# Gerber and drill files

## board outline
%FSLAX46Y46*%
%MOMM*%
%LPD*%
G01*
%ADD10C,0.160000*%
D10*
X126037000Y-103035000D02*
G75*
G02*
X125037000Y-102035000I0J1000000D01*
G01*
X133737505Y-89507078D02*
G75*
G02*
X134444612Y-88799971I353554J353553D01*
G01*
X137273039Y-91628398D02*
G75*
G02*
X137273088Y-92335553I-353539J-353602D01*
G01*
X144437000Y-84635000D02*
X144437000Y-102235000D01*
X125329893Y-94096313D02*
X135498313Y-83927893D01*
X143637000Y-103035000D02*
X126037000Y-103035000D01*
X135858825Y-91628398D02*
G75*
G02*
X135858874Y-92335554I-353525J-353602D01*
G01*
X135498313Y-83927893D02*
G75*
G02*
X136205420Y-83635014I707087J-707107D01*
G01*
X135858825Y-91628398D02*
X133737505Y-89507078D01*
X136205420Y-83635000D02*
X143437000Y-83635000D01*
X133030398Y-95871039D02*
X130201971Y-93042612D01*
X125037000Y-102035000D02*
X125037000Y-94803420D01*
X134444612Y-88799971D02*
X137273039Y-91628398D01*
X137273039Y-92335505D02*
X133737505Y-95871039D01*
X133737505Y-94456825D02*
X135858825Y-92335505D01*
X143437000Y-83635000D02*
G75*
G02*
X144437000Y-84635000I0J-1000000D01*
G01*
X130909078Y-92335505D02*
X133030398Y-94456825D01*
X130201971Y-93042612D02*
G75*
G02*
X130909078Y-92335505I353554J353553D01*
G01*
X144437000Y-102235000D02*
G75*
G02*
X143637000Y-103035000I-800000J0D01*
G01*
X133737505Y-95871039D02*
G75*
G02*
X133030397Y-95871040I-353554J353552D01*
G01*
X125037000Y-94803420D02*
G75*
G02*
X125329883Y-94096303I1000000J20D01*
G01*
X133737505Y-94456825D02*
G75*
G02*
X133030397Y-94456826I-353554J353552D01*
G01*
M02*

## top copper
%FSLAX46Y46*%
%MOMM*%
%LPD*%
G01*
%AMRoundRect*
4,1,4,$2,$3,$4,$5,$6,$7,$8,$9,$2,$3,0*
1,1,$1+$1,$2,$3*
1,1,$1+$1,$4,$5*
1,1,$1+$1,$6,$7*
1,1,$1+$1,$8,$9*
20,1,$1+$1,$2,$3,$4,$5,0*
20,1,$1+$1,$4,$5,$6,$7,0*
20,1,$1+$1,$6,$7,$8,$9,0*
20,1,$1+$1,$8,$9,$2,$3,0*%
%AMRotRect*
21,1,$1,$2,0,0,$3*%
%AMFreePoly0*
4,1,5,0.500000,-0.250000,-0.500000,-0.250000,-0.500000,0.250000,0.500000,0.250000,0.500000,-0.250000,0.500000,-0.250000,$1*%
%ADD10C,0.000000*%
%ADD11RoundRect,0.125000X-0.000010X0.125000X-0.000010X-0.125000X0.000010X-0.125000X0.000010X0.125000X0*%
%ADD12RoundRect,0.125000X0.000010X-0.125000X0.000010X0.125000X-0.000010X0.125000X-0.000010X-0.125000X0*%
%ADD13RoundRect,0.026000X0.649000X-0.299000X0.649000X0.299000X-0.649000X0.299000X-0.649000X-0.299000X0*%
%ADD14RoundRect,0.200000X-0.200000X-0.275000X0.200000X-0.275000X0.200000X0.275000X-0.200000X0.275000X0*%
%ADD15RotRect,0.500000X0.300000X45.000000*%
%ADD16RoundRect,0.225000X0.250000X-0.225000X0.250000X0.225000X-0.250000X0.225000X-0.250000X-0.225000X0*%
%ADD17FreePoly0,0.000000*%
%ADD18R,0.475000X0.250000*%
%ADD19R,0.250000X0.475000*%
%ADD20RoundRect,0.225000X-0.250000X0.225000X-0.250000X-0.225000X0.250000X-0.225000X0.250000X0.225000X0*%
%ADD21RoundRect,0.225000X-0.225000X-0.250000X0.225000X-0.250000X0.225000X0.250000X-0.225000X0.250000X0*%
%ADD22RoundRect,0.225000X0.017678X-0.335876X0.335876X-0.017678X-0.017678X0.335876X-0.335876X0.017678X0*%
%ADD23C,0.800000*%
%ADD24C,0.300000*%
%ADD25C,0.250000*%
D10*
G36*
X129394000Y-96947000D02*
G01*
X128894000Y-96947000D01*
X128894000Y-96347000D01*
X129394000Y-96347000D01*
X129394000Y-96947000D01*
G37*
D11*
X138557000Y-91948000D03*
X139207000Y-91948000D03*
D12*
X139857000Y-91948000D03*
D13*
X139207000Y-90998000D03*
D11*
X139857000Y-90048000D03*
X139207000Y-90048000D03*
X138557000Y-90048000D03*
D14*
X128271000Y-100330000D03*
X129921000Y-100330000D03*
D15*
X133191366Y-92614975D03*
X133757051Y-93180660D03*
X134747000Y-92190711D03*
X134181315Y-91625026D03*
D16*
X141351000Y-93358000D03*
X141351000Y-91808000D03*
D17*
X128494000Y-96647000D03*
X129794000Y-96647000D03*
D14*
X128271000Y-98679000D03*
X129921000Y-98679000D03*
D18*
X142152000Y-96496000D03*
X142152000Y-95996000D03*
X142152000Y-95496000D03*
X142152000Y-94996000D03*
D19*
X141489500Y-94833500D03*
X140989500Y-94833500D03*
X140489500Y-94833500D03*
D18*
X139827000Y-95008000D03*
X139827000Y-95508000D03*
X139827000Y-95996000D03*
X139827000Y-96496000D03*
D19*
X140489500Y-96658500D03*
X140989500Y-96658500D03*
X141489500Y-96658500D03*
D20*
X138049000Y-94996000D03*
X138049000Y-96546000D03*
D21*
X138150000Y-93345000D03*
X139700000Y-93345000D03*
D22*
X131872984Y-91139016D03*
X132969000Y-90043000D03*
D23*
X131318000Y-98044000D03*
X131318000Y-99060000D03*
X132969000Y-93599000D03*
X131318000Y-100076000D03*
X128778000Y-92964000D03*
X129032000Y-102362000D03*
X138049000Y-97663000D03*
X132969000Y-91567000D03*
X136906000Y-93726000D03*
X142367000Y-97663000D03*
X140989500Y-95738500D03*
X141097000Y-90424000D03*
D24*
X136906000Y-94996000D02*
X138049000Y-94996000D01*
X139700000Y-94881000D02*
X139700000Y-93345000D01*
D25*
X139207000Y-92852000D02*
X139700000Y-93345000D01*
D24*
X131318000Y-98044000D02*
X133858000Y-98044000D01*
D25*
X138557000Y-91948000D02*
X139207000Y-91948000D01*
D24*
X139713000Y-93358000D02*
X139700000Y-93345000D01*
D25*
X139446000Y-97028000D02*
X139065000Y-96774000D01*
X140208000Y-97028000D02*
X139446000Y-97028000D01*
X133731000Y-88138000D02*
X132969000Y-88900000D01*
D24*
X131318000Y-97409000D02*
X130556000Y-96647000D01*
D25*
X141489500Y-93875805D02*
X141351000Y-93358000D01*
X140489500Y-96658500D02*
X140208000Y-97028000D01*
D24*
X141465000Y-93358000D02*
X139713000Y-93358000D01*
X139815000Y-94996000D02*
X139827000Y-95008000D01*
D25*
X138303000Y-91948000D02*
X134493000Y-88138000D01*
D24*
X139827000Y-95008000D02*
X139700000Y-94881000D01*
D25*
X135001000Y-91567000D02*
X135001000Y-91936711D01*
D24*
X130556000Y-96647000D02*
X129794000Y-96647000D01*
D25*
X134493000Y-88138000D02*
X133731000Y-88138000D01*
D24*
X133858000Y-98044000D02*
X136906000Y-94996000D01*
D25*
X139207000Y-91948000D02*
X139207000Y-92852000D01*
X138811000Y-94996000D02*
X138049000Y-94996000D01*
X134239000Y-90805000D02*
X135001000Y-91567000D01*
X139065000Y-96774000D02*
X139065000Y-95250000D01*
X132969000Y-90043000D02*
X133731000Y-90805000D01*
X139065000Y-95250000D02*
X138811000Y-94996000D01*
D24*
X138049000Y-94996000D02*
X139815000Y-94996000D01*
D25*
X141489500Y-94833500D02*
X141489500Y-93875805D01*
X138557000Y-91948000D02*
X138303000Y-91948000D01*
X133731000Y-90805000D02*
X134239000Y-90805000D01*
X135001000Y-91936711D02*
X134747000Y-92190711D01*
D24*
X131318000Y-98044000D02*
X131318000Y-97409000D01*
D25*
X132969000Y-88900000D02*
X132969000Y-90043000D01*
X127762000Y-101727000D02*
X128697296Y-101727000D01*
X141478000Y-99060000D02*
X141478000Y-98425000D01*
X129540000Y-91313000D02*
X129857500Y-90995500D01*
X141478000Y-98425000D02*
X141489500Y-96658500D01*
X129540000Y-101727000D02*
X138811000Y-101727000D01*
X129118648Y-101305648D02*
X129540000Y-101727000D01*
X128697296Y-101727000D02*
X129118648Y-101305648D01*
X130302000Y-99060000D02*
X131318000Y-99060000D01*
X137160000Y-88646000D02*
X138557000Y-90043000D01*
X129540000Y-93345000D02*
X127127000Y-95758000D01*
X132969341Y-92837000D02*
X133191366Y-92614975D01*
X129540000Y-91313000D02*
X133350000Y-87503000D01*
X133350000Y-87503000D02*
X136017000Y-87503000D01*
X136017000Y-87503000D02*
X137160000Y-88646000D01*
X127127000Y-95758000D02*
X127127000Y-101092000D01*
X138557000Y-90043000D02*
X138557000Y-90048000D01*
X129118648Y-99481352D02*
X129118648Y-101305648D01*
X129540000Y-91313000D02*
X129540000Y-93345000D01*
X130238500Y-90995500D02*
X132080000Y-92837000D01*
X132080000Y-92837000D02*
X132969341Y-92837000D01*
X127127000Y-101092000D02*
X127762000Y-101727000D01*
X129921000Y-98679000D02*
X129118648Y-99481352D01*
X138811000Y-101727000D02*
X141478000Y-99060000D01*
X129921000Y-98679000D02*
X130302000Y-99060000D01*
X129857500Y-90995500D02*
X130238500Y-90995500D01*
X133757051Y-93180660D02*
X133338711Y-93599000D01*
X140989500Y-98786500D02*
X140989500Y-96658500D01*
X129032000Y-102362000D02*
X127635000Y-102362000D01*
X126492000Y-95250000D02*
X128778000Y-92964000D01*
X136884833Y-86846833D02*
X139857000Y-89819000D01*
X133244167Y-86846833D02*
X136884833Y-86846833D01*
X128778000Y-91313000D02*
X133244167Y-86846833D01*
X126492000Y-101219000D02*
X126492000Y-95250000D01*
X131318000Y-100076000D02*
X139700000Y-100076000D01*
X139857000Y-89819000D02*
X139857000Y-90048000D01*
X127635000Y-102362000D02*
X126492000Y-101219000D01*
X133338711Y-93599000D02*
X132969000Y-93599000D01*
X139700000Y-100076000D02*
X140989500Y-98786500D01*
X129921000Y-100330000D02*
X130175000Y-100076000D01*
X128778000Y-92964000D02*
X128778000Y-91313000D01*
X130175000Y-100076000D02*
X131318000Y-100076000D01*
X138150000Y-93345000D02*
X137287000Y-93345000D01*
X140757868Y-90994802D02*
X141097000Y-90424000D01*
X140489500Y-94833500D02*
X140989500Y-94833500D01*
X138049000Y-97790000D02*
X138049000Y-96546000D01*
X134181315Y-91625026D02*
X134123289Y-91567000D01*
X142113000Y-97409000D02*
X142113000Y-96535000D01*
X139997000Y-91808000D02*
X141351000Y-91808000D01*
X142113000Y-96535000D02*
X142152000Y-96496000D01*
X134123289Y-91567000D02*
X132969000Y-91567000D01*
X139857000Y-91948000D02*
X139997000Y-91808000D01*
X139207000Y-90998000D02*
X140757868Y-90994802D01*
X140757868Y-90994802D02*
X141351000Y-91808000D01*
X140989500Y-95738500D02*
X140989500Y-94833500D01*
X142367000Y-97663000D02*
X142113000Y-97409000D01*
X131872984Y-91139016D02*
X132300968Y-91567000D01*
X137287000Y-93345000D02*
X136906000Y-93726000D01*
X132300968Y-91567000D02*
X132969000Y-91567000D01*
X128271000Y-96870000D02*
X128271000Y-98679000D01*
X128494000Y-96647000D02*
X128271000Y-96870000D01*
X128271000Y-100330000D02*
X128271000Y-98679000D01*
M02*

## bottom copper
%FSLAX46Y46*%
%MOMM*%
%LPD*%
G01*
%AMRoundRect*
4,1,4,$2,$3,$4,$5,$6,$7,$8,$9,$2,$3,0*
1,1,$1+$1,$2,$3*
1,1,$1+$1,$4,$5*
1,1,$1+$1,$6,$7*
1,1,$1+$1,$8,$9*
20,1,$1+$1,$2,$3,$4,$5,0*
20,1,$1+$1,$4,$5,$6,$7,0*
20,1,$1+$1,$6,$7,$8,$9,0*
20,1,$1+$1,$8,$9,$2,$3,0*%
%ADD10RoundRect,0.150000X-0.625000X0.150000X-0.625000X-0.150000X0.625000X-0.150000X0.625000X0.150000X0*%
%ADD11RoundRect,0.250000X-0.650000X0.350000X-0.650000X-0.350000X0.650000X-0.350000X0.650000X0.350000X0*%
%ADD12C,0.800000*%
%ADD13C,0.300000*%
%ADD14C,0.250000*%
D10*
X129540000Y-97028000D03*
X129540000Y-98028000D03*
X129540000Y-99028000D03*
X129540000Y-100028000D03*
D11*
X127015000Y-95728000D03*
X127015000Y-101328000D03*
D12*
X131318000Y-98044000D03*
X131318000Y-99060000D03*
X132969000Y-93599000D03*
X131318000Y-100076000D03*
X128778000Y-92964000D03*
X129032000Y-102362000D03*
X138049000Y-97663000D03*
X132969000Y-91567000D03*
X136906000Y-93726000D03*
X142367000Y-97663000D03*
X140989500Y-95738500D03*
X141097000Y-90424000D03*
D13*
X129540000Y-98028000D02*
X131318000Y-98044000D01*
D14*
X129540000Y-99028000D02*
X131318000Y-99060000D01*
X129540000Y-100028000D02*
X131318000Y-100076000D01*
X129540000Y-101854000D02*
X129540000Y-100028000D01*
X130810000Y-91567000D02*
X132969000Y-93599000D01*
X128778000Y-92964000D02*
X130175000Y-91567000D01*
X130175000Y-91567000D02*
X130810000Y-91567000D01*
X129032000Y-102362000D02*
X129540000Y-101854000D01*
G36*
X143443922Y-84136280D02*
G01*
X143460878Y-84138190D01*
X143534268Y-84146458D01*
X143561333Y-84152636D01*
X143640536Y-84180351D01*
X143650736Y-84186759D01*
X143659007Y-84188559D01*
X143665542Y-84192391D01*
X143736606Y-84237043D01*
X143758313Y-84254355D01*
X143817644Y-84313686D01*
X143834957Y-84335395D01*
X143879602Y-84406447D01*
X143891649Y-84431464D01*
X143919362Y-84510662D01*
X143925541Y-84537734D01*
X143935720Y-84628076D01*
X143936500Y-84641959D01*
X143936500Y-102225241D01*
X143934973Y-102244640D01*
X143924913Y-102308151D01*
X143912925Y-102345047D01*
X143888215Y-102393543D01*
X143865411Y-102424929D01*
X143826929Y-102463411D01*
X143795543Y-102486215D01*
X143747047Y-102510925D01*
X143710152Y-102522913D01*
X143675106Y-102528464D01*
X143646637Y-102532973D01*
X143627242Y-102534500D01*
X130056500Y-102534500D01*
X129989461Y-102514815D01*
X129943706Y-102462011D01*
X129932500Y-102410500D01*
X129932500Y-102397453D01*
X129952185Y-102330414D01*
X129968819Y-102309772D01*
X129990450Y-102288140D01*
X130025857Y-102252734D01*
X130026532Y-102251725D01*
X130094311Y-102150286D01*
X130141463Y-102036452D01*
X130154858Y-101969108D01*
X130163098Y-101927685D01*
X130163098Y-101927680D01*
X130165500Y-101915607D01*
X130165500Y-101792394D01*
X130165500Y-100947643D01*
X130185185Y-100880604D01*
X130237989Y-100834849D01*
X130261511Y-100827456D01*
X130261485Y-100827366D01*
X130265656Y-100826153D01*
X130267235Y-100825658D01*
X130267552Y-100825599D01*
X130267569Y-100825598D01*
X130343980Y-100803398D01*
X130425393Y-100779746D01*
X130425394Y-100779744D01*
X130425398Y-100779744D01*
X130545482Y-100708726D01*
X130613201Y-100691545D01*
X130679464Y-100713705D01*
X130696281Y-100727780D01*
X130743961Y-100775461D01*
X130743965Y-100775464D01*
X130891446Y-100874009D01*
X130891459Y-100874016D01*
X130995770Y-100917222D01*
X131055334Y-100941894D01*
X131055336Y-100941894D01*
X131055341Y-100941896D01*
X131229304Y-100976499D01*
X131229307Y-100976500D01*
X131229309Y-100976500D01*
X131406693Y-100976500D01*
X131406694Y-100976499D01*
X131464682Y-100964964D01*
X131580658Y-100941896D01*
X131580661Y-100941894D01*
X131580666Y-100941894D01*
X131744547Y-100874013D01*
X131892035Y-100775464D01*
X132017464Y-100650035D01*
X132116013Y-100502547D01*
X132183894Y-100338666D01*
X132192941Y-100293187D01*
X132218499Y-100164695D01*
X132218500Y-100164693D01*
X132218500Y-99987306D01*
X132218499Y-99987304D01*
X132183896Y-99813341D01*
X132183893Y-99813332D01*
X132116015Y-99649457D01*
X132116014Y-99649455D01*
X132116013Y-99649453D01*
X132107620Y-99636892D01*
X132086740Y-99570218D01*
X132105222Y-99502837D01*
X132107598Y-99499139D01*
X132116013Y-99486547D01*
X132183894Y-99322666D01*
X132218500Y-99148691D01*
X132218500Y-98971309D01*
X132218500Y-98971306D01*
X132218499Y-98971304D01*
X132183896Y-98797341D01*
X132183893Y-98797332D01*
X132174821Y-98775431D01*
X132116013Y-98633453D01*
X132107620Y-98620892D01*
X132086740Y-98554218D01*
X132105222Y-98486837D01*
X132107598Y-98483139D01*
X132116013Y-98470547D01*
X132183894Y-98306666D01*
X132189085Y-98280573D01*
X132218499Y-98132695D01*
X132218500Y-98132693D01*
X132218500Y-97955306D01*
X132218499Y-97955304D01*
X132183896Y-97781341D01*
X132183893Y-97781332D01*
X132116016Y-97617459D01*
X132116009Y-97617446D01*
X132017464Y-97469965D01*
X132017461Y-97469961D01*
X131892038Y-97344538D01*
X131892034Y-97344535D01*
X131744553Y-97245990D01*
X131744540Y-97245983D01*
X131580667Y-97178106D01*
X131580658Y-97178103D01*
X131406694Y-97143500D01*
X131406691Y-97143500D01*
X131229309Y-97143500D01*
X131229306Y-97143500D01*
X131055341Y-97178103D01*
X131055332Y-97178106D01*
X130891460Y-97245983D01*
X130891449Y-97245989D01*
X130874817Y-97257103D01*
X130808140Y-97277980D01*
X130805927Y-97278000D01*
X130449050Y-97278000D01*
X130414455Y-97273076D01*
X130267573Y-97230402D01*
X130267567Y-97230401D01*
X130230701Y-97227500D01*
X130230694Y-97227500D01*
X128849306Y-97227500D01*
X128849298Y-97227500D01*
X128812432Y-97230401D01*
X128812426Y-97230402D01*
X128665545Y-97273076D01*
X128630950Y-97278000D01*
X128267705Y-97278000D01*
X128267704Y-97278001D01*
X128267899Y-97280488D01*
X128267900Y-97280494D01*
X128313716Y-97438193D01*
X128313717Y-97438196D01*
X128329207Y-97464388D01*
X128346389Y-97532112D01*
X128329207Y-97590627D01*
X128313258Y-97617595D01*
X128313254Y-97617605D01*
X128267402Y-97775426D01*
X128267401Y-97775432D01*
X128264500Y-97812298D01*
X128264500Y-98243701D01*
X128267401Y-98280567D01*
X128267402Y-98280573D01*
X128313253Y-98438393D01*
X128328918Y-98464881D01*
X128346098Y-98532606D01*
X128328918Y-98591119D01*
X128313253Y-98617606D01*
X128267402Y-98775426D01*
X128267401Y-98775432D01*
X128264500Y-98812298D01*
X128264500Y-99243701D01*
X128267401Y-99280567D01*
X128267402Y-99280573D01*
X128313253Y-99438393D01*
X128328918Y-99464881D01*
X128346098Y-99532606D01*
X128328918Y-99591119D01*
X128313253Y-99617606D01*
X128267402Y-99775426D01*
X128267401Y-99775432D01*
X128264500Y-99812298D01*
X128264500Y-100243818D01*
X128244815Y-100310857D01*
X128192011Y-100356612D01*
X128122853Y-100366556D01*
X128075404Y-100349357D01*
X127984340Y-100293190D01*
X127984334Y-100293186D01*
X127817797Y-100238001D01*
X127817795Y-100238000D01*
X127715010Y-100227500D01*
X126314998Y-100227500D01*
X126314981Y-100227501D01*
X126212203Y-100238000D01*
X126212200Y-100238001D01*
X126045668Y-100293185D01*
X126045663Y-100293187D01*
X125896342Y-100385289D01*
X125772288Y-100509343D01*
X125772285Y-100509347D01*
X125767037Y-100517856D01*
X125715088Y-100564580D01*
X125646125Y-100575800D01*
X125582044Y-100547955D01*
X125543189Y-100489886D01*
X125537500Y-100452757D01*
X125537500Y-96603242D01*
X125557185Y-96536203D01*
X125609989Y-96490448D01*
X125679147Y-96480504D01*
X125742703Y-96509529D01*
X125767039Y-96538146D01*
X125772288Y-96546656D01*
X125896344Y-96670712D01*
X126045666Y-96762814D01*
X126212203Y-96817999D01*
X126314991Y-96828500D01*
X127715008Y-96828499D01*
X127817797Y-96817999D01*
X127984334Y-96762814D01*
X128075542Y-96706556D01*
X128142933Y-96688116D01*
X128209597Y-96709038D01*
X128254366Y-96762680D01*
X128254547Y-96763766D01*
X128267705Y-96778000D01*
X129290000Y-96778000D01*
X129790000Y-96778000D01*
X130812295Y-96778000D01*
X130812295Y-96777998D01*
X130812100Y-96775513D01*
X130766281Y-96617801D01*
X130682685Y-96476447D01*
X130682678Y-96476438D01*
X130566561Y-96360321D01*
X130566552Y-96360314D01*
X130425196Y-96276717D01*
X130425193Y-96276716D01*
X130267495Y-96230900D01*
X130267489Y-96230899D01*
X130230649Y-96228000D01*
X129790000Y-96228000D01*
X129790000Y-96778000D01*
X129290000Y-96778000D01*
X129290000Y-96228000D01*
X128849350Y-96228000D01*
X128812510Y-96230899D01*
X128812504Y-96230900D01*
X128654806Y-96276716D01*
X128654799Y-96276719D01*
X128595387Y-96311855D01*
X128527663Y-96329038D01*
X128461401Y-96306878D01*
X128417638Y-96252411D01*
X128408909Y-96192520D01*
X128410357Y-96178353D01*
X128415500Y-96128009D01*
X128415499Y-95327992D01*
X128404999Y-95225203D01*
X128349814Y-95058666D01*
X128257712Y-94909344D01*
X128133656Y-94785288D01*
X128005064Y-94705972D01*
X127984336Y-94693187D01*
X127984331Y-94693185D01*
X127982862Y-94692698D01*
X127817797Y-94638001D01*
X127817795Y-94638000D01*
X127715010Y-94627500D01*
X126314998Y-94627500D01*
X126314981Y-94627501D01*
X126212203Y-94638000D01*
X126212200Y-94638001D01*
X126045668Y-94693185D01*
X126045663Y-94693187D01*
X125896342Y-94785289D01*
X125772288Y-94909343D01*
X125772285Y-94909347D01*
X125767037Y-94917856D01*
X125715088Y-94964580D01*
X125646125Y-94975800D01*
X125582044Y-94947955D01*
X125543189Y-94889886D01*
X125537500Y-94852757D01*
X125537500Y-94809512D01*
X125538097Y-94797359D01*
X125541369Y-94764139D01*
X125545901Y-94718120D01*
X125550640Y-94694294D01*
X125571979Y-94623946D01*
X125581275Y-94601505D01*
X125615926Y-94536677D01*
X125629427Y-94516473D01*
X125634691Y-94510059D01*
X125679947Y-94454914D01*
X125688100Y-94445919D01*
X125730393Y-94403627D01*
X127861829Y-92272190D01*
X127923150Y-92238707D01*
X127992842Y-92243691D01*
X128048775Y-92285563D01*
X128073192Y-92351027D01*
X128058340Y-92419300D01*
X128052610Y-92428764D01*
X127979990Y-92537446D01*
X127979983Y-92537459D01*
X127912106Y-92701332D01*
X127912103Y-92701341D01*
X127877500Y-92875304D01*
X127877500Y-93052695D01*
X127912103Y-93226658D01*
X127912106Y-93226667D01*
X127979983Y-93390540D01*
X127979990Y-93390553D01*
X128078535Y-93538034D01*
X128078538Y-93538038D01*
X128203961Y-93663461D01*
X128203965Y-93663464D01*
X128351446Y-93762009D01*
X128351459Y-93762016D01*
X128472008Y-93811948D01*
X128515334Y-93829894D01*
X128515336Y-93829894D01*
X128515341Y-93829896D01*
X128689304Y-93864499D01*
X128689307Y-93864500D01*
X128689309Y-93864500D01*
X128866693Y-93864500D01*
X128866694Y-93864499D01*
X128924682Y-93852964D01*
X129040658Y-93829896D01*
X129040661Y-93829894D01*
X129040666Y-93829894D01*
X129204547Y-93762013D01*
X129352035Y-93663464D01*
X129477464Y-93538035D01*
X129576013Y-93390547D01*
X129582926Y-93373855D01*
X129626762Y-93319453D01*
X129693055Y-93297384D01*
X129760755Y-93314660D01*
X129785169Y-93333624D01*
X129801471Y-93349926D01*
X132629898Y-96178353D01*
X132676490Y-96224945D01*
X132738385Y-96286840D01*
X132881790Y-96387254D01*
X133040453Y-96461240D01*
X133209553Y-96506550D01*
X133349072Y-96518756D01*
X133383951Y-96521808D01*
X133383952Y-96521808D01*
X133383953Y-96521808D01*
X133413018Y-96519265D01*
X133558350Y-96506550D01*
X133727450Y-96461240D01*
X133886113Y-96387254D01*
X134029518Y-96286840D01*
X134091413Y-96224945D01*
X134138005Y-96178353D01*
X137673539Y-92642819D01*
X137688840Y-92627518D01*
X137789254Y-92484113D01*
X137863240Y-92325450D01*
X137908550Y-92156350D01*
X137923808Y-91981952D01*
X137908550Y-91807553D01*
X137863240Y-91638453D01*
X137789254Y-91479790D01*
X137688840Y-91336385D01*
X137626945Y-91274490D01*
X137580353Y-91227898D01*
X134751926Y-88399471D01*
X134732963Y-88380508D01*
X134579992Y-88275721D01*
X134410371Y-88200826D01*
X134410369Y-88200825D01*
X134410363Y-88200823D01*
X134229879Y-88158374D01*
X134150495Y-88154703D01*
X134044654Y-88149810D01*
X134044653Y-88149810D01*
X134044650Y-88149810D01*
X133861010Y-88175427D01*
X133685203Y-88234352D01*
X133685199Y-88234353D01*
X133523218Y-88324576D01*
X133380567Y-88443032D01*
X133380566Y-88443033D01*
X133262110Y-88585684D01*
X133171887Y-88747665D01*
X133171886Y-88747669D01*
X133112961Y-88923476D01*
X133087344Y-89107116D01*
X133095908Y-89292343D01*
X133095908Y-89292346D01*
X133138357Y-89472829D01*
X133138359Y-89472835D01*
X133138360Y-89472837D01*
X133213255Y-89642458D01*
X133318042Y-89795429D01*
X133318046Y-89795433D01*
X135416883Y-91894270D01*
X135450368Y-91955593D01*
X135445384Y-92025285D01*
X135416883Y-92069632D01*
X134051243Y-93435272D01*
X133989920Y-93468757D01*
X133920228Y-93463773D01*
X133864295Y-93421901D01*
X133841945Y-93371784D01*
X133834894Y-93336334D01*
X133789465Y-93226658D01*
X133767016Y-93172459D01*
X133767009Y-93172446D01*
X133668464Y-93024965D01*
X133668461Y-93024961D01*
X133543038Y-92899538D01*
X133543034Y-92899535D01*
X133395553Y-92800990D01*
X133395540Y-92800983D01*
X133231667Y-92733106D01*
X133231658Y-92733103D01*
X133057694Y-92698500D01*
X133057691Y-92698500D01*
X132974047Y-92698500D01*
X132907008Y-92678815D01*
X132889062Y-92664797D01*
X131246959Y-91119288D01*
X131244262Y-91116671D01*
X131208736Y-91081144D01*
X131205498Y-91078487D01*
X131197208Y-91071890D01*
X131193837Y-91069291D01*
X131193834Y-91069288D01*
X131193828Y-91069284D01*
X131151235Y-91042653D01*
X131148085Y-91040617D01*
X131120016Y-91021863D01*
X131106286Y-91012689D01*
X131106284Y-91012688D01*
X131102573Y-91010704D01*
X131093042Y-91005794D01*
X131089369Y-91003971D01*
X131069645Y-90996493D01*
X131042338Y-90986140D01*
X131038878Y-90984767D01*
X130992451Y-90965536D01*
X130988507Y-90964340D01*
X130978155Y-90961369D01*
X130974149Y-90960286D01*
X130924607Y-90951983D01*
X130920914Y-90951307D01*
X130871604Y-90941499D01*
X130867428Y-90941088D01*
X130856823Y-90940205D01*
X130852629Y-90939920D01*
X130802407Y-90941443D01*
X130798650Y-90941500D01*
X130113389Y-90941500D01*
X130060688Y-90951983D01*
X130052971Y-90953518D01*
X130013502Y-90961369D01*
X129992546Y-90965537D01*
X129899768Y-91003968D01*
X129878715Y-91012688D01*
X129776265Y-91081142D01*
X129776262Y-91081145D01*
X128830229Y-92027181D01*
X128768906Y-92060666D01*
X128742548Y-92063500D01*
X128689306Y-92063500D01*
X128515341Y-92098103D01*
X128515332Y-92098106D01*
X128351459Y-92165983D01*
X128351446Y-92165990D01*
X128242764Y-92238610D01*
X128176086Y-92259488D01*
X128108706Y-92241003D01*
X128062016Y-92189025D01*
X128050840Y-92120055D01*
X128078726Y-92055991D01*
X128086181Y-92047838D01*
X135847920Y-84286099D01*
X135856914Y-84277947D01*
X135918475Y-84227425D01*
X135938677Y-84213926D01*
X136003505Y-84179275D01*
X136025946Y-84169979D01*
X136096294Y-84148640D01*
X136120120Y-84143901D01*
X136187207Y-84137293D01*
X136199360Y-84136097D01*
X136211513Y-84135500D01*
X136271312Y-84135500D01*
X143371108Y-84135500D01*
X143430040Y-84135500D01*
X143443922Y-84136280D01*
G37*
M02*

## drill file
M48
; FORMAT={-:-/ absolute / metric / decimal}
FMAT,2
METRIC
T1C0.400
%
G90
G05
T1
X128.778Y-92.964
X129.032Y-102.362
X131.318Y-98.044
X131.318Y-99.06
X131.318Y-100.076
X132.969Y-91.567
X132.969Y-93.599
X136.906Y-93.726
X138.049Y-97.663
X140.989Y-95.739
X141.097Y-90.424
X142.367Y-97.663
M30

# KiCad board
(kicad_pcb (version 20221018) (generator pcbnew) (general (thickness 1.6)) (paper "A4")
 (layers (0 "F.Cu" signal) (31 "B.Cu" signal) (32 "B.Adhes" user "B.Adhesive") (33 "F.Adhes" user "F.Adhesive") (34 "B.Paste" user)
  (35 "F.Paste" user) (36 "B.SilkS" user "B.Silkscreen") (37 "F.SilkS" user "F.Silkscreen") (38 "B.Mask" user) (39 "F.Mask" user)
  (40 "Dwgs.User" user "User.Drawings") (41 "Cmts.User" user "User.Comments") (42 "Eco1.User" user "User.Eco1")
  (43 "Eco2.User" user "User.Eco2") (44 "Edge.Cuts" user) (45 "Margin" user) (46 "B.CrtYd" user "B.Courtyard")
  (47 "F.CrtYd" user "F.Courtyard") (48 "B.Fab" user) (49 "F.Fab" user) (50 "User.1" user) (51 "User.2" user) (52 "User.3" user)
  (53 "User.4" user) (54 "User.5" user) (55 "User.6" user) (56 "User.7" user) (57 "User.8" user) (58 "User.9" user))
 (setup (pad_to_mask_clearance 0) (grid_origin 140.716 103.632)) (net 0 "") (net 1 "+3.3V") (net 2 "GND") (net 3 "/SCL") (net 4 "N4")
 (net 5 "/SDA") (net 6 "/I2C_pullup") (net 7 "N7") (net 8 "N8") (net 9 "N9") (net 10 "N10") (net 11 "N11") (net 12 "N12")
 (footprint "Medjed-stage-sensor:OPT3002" (layer "F.Cu") (at 139.207 90.998 90)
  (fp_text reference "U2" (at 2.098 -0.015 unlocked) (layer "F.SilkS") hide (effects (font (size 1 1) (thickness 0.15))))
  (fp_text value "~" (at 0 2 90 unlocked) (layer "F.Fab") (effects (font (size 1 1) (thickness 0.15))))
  (pad "1" smd roundrect (at -0.95 -0.65 270) (size 0.5 0.25) (layers "F.Cu" "F.Paste" "F.Mask") (roundrect_rratio 0.5) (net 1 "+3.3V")
   (thermal_bridge_angle 45))
  (pad "2" smd roundrect (at -0.95 0 270) (size 0.5 0.25) (layers "F.Cu" "F.Paste" "F.Mask") (roundrect_rratio 0.5) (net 1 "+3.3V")
   (thermal_bridge_angle 45))
  (pad "3" smd roundrect (at -0.95 0.65 90) (size 0.5 0.25) (layers "F.Cu" "F.Paste" "F.Mask") (roundrect_rratio 0.5) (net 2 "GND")
   (thermal_bridge_angle 45))
  (pad "3" smd roundrect (at 0 0 90) (size 0.65 1.35) (layers "F.Cu" "F.Paste" "F.Mask") (roundrect_rratio 0.04) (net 2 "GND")
   (thermal_bridge_angle 45))
  (pad "4" smd roundrect (at 0.95 0.65 270) (size 0.5 0.25) (layers "F.Cu" "F.Paste" "F.Mask") (roundrect_rratio 0.5) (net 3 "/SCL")
   (thermal_bridge_angle 45))
  (pad "5" smd roundrect (at 0.95 0 270) (size 0.5 0.25) (layers "F.Cu" "F.Paste" "F.Mask") (roundrect_rratio 0.5) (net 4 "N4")
   (thermal_bridge_angle 45))
  (pad "6" smd roundrect (at 0.95 -0.65 270) (size 0.5 0.25) (layers "F.Cu" "F.Paste" "F.Mask") (roundrect_rratio 0.5) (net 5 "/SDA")
   (thermal_bridge_angle 45)))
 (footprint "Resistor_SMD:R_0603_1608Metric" (layer "F.Cu") (at 129.096 100.33)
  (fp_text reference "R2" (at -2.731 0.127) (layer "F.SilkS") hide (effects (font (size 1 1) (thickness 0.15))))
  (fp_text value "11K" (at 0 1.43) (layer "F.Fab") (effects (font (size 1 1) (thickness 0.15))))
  (pad "1" smd roundrect (at -0.825 0) (size 0.8 0.95) (layers "F.Cu" "F.Paste" "F.Mask") (roundrect_rratio 0.25) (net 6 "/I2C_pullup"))
  (pad "2" smd roundrect (at 0.825 0) (size 0.8 0.95) (layers "F.Cu" "F.Paste" "F.Mask") (roundrect_rratio 0.25) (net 3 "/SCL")))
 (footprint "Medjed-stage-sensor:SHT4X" (layer "F.Cu") (at 133.969183 92.402843 45)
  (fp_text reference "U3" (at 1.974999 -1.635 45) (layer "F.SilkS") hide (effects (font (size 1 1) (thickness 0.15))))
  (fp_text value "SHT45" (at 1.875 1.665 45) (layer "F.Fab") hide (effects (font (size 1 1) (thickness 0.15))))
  (pad "1" smd rect (at -0.7 -0.4 45) (size 0.5 0.3) (layers "F.Cu" "F.Paste" "F.Mask") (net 5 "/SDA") (solder_mask_margin 0.102))
  (pad "2" smd rect (at -0.7 0.4 45) (size 0.5 0.3) (layers "F.Cu" "F.Paste" "F.Mask") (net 3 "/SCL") (solder_mask_margin 0.102))
  (pad "3" smd rect (at 0.7 0.4 45) (size 0.5 0.3) (layers "F.Cu" "F.Paste" "F.Mask") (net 1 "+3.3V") (solder_mask_margin 0.102))
  (pad "4" smd rect (at 0.7 -0.4 45) (size 0.5 0.3) (layers "F.Cu" "F.Paste" "F.Mask") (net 2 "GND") (solder_mask_margin 0.102)))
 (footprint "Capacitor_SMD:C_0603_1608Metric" (layer "F.Cu") (at 141.351 92.583 90)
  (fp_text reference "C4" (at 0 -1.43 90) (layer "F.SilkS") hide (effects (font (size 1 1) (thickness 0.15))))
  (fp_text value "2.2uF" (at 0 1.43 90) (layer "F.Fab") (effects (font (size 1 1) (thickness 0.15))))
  (pad "1" smd roundrect (at -0.775 0 90) (size 0.9 0.95) (layers "F.Cu" "F.Paste" "F.Mask") (roundrect_rratio 0.25) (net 1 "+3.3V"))
  (pad "2" smd roundrect (at 0.775 0 90) (size 0.9 0.95) (layers "F.Cu" "F.Paste" "F.Mask") (roundrect_rratio 0.25) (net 2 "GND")))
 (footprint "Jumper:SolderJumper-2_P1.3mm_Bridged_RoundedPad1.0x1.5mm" (layer "F.Cu") (at 129.144 96.647) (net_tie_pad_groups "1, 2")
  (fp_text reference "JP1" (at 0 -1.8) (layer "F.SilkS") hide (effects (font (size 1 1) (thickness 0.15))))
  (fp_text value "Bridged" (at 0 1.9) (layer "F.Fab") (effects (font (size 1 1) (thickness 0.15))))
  (fp_poly (pts (xy 0.25 -0.3) (xy -0.25 -0.3) (xy -0.25 0.3) (xy 0.25 0.3)) (stroke (width 0) (type solid)) (fill solid) (layer "F.Cu"))
  (pad "1" smd custom (at -0.65 0) (size 1 0.5) (layers "F.Cu" "F.Mask") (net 6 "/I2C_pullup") (zone_connect 2) (thermal_bridge_angle 45)
   (options (clearance outline) (anchor rect)) (primitives))
  (pad "2" smd custom (at 0.65 0) (size 1 0.5) (layers "F.Cu" "F.Mask") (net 1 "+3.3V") (zone_connect 2) (thermal_bridge_angle 45)
   (options (clearance outline) (anchor rect)) (primitives)))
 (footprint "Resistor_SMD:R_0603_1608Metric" (layer "F.Cu") (at 129.096 98.679)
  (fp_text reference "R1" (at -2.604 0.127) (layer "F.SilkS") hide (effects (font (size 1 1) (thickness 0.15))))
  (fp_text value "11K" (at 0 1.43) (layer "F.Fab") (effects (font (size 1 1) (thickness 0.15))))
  (pad "1" smd roundrect (at -0.825 0) (size 0.8 0.95) (layers "F.Cu" "F.Paste" "F.Mask") (roundrect_rratio 0.25) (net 6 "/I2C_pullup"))
  (pad "2" smd roundrect (at 0.825 0) (size 0.8 0.95) (layers "F.Cu" "F.Paste" "F.Mask") (roundrect_rratio 0.25) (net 5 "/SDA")))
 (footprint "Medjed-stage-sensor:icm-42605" (layer "F.Cu") (at 140.9895 95.746 180)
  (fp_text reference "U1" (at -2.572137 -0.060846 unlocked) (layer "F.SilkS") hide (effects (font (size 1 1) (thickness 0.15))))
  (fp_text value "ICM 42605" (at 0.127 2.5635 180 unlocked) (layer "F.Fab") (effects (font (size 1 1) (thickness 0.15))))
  (pad "1" smd rect (at -1.1625 -0.75 270) (size 0.25 0.475) (layers "F.Cu" "F.Paste" "F.Mask") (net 2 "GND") (thermal_bridge_angle 45))
  (pad "2" smd rect (at -1.1625 -0.25 270) (size 0.25 0.475) (layers "F.Cu" "F.Paste" "F.Mask") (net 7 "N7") (thermal_bridge_angle 45))
  (pad "3" smd rect (at -1.1625 0.25 270) (size 0.25 0.475) (layers "F.Cu" "F.Paste" "F.Mask") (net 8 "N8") (thermal_bridge_angle 45))
  (pad "4" smd rect (at -1.1625 0.75 270) (size 0.25 0.475) (layers "F.Cu" "F.Paste" "F.Mask") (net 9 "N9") (thermal_bridge_angle 45))
  (pad "5" smd rect (at -0.5 0.9125 180) (size 0.25 0.475) (layers "F.Cu" "F.Paste" "F.Mask") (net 1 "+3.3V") (thermal_bridge_angle 45))
  (pad "6" smd rect (at 0 0.9125 180) (size 0.25 0.475) (layers "F.Cu" "F.Paste" "F.Mask") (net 2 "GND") (thermal_bridge_angle 45))
  (pad "7" smd rect (at 0.5 0.9125 180) (size 0.25 0.475) (layers "F.Cu" "F.Paste" "F.Mask") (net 2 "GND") (thermal_bridge_angle 45))
  (pad "8" smd rect (at 1.1625 0.738 270) (size 0.25 0.475) (layers "F.Cu" "F.Paste" "F.Mask") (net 1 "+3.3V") (thermal_bridge_angle 45))
  (pad "9" smd rect (at 1.1625 0.238 270) (size 0.25 0.475) (layers "F.Cu" "F.Paste" "F.Mask") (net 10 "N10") (thermal_bridge_angle 45))
  (pad "10" smd rect (at 1.1625 -0.25 270) (size 0.25 0.475) (layers "F.Cu" "F.Paste" "F.Mask") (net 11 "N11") (thermal_bridge_angle 45))
  (pad "11" smd rect (at 1.1625 -0.75 270) (size 0.25 0.475) (layers "F.Cu" "F.Paste" "F.Mask") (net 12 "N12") (thermal_bridge_angle 45))
  (pad "12" smd rect (at 0.5 -0.9125 180) (size 0.25 0.475) (layers "F.Cu" "F.Paste" "F.Mask") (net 1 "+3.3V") (thermal_bridge_angle 45))
  (pad "13" smd rect (at 0 -0.9125 180) (size 0.25 0.475) (layers "F.Cu" "F.Paste" "F.Mask") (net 3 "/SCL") (thermal_bridge_angle 45))
  (pad "14" smd rect (at -0.5 -0.9125 180) (size 0.25 0.475) (layers "F.Cu" "F.Paste" "F.Mask") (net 5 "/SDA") (thermal_bridge_angle 45)))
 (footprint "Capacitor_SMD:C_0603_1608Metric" (layer "F.Cu") (at 138.049 95.771 -90)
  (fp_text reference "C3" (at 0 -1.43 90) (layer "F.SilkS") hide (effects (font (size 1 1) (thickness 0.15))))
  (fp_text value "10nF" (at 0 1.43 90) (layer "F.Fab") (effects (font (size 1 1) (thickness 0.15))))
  (pad "1" smd roundrect (at -0.775 0 270) (size 0.9 0.95) (layers "F.Cu" "F.Paste" "F.Mask") (roundrect_rratio 0.25) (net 1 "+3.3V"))
  (pad "2" smd roundrect (at 0.775 0 270) (size 0.9 0.95) (layers "F.Cu" "F.Paste" "F.Mask") (roundrect_rratio 0.25) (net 2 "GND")))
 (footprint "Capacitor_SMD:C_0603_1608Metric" (layer "F.Cu") (at 138.925 93.345)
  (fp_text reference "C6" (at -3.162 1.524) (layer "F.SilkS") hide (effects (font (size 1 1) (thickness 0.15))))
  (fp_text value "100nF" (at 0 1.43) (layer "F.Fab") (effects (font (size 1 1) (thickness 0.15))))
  (pad "1" smd roundrect (at -0.775 0) (size 0.9 0.95) (layers "F.Cu" "F.Paste" "F.Mask") (roundrect_rratio 0.25) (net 2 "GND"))
  (pad "2" smd roundrect (at 0.775 0) (size 0.9 0.95) (layers "F.Cu" "F.Paste" "F.Mask") (roundrect_rratio 0.25) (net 1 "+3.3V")))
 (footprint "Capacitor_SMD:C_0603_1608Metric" (layer "F.Cu") (at 132.420992 90.591008 45)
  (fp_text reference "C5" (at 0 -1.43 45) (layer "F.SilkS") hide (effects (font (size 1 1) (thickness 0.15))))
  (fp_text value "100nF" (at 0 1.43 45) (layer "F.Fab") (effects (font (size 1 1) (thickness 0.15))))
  (pad "1" smd roundrect (at -0.775 0 45) (size 0.9 0.95) (layers "F.Cu" "F.Paste" "F.Mask") (roundrect_rratio 0.25) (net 2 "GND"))
  (pad "2" smd roundrect (at 0.775 0 45) (size 0.9 0.95) (layers "F.Cu" "F.Paste" "F.Mask") (roundrect_rratio 0.25) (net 1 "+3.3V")))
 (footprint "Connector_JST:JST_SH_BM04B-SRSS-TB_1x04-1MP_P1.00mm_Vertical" (layer "B.Cu") (at 128.215 98.528 -90)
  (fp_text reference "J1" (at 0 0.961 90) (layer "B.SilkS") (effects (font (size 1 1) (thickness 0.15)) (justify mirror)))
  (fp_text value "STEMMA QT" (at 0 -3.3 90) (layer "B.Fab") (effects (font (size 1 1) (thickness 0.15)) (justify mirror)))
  (pad "1" smd roundrect (at -1.5 -1.325 270) (size 0.6 1.55) (layers "B.Cu" "B.Paste" "B.Mask") (roundrect_rratio 0.25) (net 2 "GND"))
  (pad "2" smd roundrect (at -0.5 -1.325 270) (size 0.6 1.55) (layers "B.Cu" "B.Paste" "B.Mask") (roundrect_rratio 0.25) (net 1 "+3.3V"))
  (pad "3" smd roundrect (at 0.5 -1.325 270) (size 0.6 1.55) (layers "B.Cu" "B.Paste" "B.Mask") (roundrect_rratio 0.25) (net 5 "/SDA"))
  (pad "4" smd roundrect (at 1.5 -1.325 270) (size 0.6 1.55) (layers "B.Cu" "B.Paste" "B.Mask") (roundrect_rratio 0.25) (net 3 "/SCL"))
  (pad "MP" smd roundrect (at -2.8 1.2 270) (size 1.2 1.8) (layers "B.Cu" "B.Paste" "B.Mask") (roundrect_rratio 0.208333))
  (pad "MP" smd roundrect (at 2.8 1.2 270) (size 1.2 1.8) (layers "B.Cu" "B.Paste" "B.Mask") (roundrect_rratio 0.208333)))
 (gr_arc (start 126.037 103.035) (mid 125.329893 102.742107) (end 125.037 102.035) (stroke (width 0.16) (type solid)) (layer "Edge.Cuts"))
 (gr_arc (start 133.737505 89.507078) (mid 133.737505 88.799971) (end 134.444612 88.799971) (stroke (width 0.16) (type solid))
  (layer "Edge.Cuts"))
 (gr_arc (start 137.273039 91.628398) (mid 137.419486 91.981952) (end 137.273039 92.335505) (stroke (width 0.16) (type solid))
  (layer "Edge.Cuts"))
 (gr_line (start 144.437 84.635) (end 144.437 102.235) (stroke (width 0.16) (type solid)) (layer "Edge.Cuts"))
 (gr_line (start 125.329893 94.096313) (end 135.498313 83.927893) (stroke (width 0.16) (type solid)) (layer "Edge.Cuts"))
 (gr_line (start 143.637 103.035) (end 126.037 103.035) (stroke (width 0.16) (type solid)) (layer "Edge.Cuts"))
 (gr_arc (start 135.858825 91.628398) (mid 136.005272 91.981952) (end 135.858825 92.335505) (stroke (width 0.16) (type solid))
  (layer "Edge.Cuts"))
 (gr_arc (start 135.498313 83.927893) (mid 135.822737 83.71112) (end 136.20542 83.635) (stroke (width 0.16) (type solid))
  (layer "Edge.Cuts"))
 (gr_line (start 135.858825 91.628398) (end 133.737505 89.507078) (stroke (width 0.16) (type solid)) (layer "Edge.Cuts"))
 (gr_line (start 136.20542 83.635) (end 143.437 83.635) (stroke (width 0.16) (type solid)) (layer "Edge.Cuts"))
 (gr_line (start 133.030398 95.871039) (end 130.201971 93.042612) (stroke (width 0.16) (type solid)) (layer "Edge.Cuts"))
 (gr_line (start 125.037 102.035) (end 125.037 94.80342) (stroke (width 0.16) (type solid)) (layer "Edge.Cuts"))
 (gr_line (start 134.444612 88.799971) (end 137.273039 91.628398) (stroke (width 0.16) (type solid)) (layer "Edge.Cuts"))
 (gr_line (start 137.273039 92.335505) (end 133.737505 95.871039) (stroke (width 0.16) (type solid)) (layer "Edge.Cuts"))
 (gr_line (start 133.737505 94.456825) (end 135.858825 92.335505) (stroke (width 0.16) (type solid)) (layer "Edge.Cuts"))
 (gr_arc (start 143.437 83.635) (mid 144.144107 83.927893) (end 144.437 84.635) (stroke (width 0.16) (type solid)) (layer "Edge.Cuts"))
 (gr_line (start 130.909078 92.335505) (end 133.030398 94.456825) (stroke (width 0.16) (type solid)) (layer "Edge.Cuts"))
 (gr_arc (start 130.201971 93.042612) (mid 130.201971 92.335505) (end 130.909078 92.335505) (stroke (width 0.16) (type solid))
  (layer "Edge.Cuts"))
 (gr_arc (start 144.437 102.235) (mid 144.202685 102.800685) (end 143.637 103.035) (stroke (width 0.16) (type solid)) (layer "Edge.Cuts"))
 (gr_arc (start 133.737505 95.871039) (mid 133.383952 96.017486) (end 133.030398 95.871039) (stroke (width 0.16) (type solid))
  (layer "Edge.Cuts"))
 (gr_arc (start 125.037 94.80342) (mid 125.11312 94.420737) (end 125.329893 94.096313) (stroke (width 0.16) (type solid))
  (layer "Edge.Cuts"))
 (gr_arc (start 133.737505 94.456825) (mid 133.383952 94.603272) (end 133.030398 94.456825) (stroke (width 0.16) (type solid))
  (layer "Edge.Cuts"))
 (segment (start 136.906 94.996) (end 138.049 94.996) (width 0.3) (layer "F.Cu") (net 1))
 (segment (start 139.7 94.881) (end 139.7 93.345) (width 0.3) (layer "F.Cu") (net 1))
 (segment (start 139.207 92.852) (end 139.7 93.345) (width 0.25) (layer "F.Cu") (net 1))
 (segment (start 131.318 98.044) (end 133.858 98.044) (width 0.3) (layer "F.Cu") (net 1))
 (segment (start 138.557 91.948) (end 139.207 91.948) (width 0.25) (layer "F.Cu") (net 1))
 (segment (start 139.713 93.358) (end 139.7 93.345) (width 0.3) (layer "F.Cu") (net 1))
 (segment (start 139.446 97.028) (end 139.065 96.774) (width 0.25) (layer "F.Cu") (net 1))
 (segment (start 140.208 97.028) (end 139.446 97.028) (width 0.25) (layer "F.Cu") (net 1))
 (segment (start 133.731 88.138) (end 132.969 88.9) (width 0.25) (layer "F.Cu") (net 1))
 (segment (start 131.318 97.409) (end 130.556 96.647) (width 0.3) (layer "F.Cu") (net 1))
 (segment (start 141.4895 93.875805) (end 141.351 93.358) (width 0.25) (layer "F.Cu") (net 1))
 (segment (start 140.4895 96.6585) (end 140.208 97.028) (width 0.25) (layer "F.Cu") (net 1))
 (segment (start 141.465 93.358) (end 139.713 93.358) (width 0.3) (layer "F.Cu") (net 1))
 (segment (start 139.815 94.996) (end 139.827 95.008) (width 0.3) (layer "F.Cu") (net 1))
 (segment (start 138.303 91.948) (end 134.493 88.138) (width 0.25) (layer "F.Cu") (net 1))
 (segment (start 139.827 95.008) (end 139.7 94.881) (width 0.3) (layer "F.Cu") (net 1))
 (segment (start 135.001 91.567) (end 135.001 91.936711) (width 0.25) (layer "F.Cu") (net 1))
 (segment (start 130.556 96.647) (end 129.794 96.647) (width 0.3) (layer "F.Cu") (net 1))
 (segment (start 134.493 88.138) (end 133.731 88.138) (width 0.25) (layer "F.Cu") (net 1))
 (segment (start 133.858 98.044) (end 136.906 94.996) (width 0.3) (layer "F.Cu") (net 1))
 (segment (start 139.207 91.948) (end 139.207 92.852) (width 0.25) (layer "F.Cu") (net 1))
 (segment (start 138.811 94.996) (end 138.049 94.996) (width 0.25) (layer "F.Cu") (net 1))
 (segment (start 134.239 90.805) (end 135.001 91.567) (width 0.25) (layer "F.Cu") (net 1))
 (segment (start 139.065 96.774) (end 139.065 95.25) (width 0.25) (layer "F.Cu") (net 1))
 (segment (start 132.969 90.043) (end 133.731 90.805) (width 0.25) (layer "F.Cu") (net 1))
 (segment (start 139.065 95.25) (end 138.811 94.996) (width 0.25) (layer "F.Cu") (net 1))
 (segment (start 138.049 94.996) (end 139.815 94.996) (width 0.3) (layer "F.Cu") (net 1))
 (segment (start 141.4895 94.8335) (end 141.4895 93.875805) (width 0.25) (layer "F.Cu") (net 1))
 (segment (start 138.557 91.948) (end 138.303 91.948) (width 0.25) (layer "F.Cu") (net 1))
 (segment (start 133.731 90.805) (end 134.239 90.805) (width 0.25) (layer "F.Cu") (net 1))
 (segment (start 135.001 91.936711) (end 134.747 92.190711) (width 0.25) (layer "F.Cu") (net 1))
 (segment (start 131.318 98.044) (end 131.318 97.409) (width 0.3) (layer "F.Cu") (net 1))
 (segment (start 132.969 88.9) (end 132.969 90.043) (width 0.25) (layer "F.Cu") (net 1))
 (via (at 131.318 98.044) (size 0.8) (drill 0.4) (layers "F.Cu" "B.Cu") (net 1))
 (segment (start 129.54 98.028) (end 131.318 98.044) (width 0.3) (layer "B.Cu") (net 1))
 (segment (start 127.762 101.727) (end 128.697296 101.727) (width 0.25) (layer "F.Cu") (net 5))
 (segment (start 141.478 99.06) (end 141.478 98.425) (width 0.25) (layer "F.Cu") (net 5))
 (segment (start 129.54 91.313) (end 129.8575 90.9955) (width 0.25) (layer "F.Cu") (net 5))
 (segment (start 141.478 98.425) (end 141.4895 96.6585) (width 0.25) (layer "F.Cu") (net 5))
 (segment (start 129.54 101.727) (end 138.811 101.727) (width 0.25) (layer "F.Cu") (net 5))
 (segment (start 129.118648 101.305648) (end 129.54 101.727) (width 0.25) (layer "F.Cu") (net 5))
 (segment (start 128.697296 101.727) (end 129.118648 101.305648) (width 0.25) (layer "F.Cu") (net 5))
 (segment (start 130.302 99.06) (end 131.318 99.06) (width 0.25) (layer "F.Cu") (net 5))
 (segment (start 137.16 88.646) (end 138.557 90.043) (width 0.25) (layer "F.Cu") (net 5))
 (segment (start 129.54 93.345) (end 127.127 95.758) (width 0.25) (layer "F.Cu") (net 5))
 (segment (start 132.969341 92.837) (end 133.191366 92.614975) (width 0.25) (layer "F.Cu") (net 5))
 (segment (start 129.54 91.313) (end 133.35 87.503) (width 0.25) (layer "F.Cu") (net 5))
 (segment (start 133.35 87.503) (end 136.017 87.503) (width 0.25) (layer "F.Cu") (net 5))
 (segment (start 136.017 87.503) (end 137.16 88.646) (width 0.25) (layer "F.Cu") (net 5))
 (segment (start 127.127 95.758) (end 127.127 101.092) (width 0.25) (layer "F.Cu") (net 5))
 (segment (start 138.557 90.043) (end 138.557 90.048) (width 0.25) (layer "F.Cu") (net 5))
 (segment (start 129.118648 99.481352) (end 129.118648 101.305648) (width 0.25) (layer "F.Cu") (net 5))
 (segment (start 129.54 91.313) (end 129.54 93.345) (width 0.25) (layer "F.Cu") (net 5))
 (segment (start 130.2385 90.9955) (end 132.08 92.837) (width 0.25) (layer "F.Cu") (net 5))
 (segment (start 132.08 92.837) (end 132.969341 92.837) (width 0.25) (layer "F.Cu") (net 5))
 (segment (start 127.127 101.092) (end 127.762 101.727) (width 0.25) (layer "F.Cu") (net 5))
 (segment (start 129.921 98.679) (end 129.118648 99.481352) (width 0.25) (layer "F.Cu") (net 5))
 (segment (start 138.811 101.727) (end 141.478 99.06) (width 0.25) (layer "F.Cu") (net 5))
 (segment (start 129.921 98.679) (end 130.302 99.06) (width 0.25) (layer "F.Cu") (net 5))
 (segment (start 129.8575 90.9955) (end 130.2385 90.9955) (width 0.25) (layer "F.Cu") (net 5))
 (via (at 131.318 99.06) (size 0.8) (drill 0.4) (layers "F.Cu" "B.Cu") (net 5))
 (segment (start 129.54 99.028) (end 131.318 99.06) (width 0.25) (layer "B.Cu") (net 5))
 (segment (start 133.757051 93.18066) (end 133.338711 93.599) (width 0.25) (layer "F.Cu") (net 3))
 (segment (start 140.9895 98.7865) (end 140.9895 96.6585) (width 0.25) (layer "F.Cu") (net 3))
 (segment (start 129.032 102.362) (end 127.635 102.362) (width 0.25) (layer "F.Cu") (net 3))
 (segment (start 126.492 95.25) (end 128.778 92.964) (width 0.25) (layer "F.Cu") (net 3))
 (segment (start 136.884833 86.846833) (end 139.857 89.819) (width 0.25) (layer "F.Cu") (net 3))
 (segment (start 133.244167 86.846833) (end 136.884833 86.846833) (width 0.25) (layer "F.Cu") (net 3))
 (segment (start 128.778 91.313) (end 133.244167 86.846833) (width 0.25) (layer "F.Cu") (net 3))
 (segment (start 126.492 101.219) (end 126.492 95.25) (width 0.25) (layer "F.Cu") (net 3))
 (segment (start 131.318 100.076) (end 139.7 100.076) (width 0.25) (layer "F.Cu") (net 3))
 (segment (start 139.857 89.819) (end 139.857 90.048) (width 0.25) (layer "F.Cu") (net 3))
 (segment (start 127.635 102.362) (end 126.492 101.219) (width 0.25) (layer "F.Cu") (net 3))
 (segment (start 133.338711 93.599) (end 132.969 93.599) (width 0.25) (layer "F.Cu") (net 3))
 (segment (start 139.7 100.076) (end 140.9895 98.7865) (width 0.25) (layer "F.Cu") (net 3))
 (segment (start 129.921 100.33) (end 130.175 100.076) (width 0.25) (layer "F.Cu") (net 3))
 (segment (start 128.778 92.964) (end 128.778 91.313) (width 0.25) (layer "F.Cu") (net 3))
 (segment (start 130.175 100.076) (end 131.318 100.076) (width 0.25) (layer "F.Cu") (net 3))
 (via (at 132.969 93.599) (size 0.8) (drill 0.4) (layers "F.Cu" "B.Cu") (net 3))
 (via (at 131.318 100.076) (size 0.8) (drill 0.4) (layers "F.Cu" "B.Cu") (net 3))
 (via (at 128.778 92.964) (size 0.8) (drill 0.4) (layers "F.Cu" "B.Cu") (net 3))
 (via (at 129.032 102.362) (size 0.8) (drill 0.4) (layers "F.Cu" "B.Cu") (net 3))
 (segment (start 129.54 100.028) (end 131.318 100.076) (width 0.25) (layer "B.Cu") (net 3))
 (segment (start 129.54 101.854) (end 129.54 100.028) (width 0.25) (layer "B.Cu") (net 3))
 (segment (start 130.81 91.567) (end 132.969 93.599) (width 0.25) (layer "B.Cu") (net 3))
 (segment (start 128.778 92.964) (end 130.175 91.567) (width 0.25) (layer "B.Cu") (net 3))
 (segment (start 130.175 91.567) (end 130.81 91.567) (width 0.25) (layer "B.Cu") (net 3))
 (segment (start 129.032 102.362) (end 129.54 101.854) (width 0.25) (layer "B.Cu") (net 3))
 (segment (start 138.15 93.345) (end 137.287 93.345) (width 0.25) (layer "F.Cu") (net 2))
 (segment (start 140.757868 90.994802) (end 141.097 90.424) (width 0.25) (layer "F.Cu") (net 2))
 (segment (start 140.4895 94.8335) (end 140.9895 94.8335) (width 0.25) (layer "F.Cu") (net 2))
 (segment (start 138.049 97.79) (end 138.049 96.546) (width 0.25) (layer "F.Cu") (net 2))
 (segment (start 134.181315 91.625026) (end 134.123289 91.567) (width 0.25) (layer "F.Cu") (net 2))
 (segment (start 142.113 97.409) (end 142.113 96.535) (width 0.25) (layer "F.Cu") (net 2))
 (segment (start 139.997 91.808) (end 141.351 91.808) (width 0.25) (layer "F.Cu") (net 2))
 (segment (start 142.113 96.535) (end 142.152 96.496) (width 0.25) (layer "F.Cu") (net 2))
 (segment (start 134.123289 91.567) (end 132.969 91.567) (width 0.25) (layer "F.Cu") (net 2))
 (segment (start 139.857 91.948) (end 139.997 91.808) (width 0.25) (layer "F.Cu") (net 2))
 (segment (start 139.207 90.998) (end 140.757868 90.994802) (width 0.25) (layer "F.Cu") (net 2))
 (segment (start 140.757868 90.994802) (end 141.351 91.808) (width 0.25) (layer "F.Cu") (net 2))
 (segment (start 140.9895 95.7385) (end 140.9895 94.8335) (width 0.25) (layer "F.Cu") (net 2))
 (segment (start 142.367 97.663) (end 142.113 97.409) (width 0.25) (layer "F.Cu") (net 2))
 (segment (start 131.872984 91.139016) (end 132.300968 91.567) (width 0.25) (layer "F.Cu") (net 2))
 (segment (start 137.287 93.345) (end 136.906 93.726) (width 0.25) (layer "F.Cu") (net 2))
 (segment (start 132.300968 91.567) (end 132.969 91.567) (width 0.25) (layer "F.Cu") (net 2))
 (via (at 138.049 97.663) (size 0.8) (drill 0.4) (layers "F.Cu" "B.Cu") (free) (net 2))
 (via (at 132.969 91.567) (size 0.8) (drill 0.4) (layers "F.Cu" "B.Cu") (free) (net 2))
 (via (at 136.906 93.726) (size 0.8) (drill 0.4) (layers "F.Cu" "B.Cu") (free) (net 2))
 (via (at 142.367 97.663) (size 0.8) (drill 0.4) (layers "F.Cu" "B.Cu") (free) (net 2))
 (via (at 140.9895 95.7385) (size 0.8) (drill 0.4) (layers "F.Cu" "B.Cu") (free) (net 2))
 (via (at 141.097 90.424) (size 0.8) (drill 0.4) (layers "F.Cu" "B.Cu") (free) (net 2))
 (segment (start 128.271 96.87) (end 128.271 98.679) (width 0.25) (layer "F.Cu") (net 6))
 (segment (start 128.494 96.647) (end 128.271 96.87) (width 0.25) (layer "F.Cu") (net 6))
 (segment (start 128.271 100.33) (end 128.271 98.679) (width 0.25) (layer "F.Cu") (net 6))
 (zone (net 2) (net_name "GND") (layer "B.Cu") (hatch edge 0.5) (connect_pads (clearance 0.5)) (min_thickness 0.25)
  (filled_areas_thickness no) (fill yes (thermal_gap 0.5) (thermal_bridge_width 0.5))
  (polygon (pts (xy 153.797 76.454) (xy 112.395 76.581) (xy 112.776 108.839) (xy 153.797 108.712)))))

